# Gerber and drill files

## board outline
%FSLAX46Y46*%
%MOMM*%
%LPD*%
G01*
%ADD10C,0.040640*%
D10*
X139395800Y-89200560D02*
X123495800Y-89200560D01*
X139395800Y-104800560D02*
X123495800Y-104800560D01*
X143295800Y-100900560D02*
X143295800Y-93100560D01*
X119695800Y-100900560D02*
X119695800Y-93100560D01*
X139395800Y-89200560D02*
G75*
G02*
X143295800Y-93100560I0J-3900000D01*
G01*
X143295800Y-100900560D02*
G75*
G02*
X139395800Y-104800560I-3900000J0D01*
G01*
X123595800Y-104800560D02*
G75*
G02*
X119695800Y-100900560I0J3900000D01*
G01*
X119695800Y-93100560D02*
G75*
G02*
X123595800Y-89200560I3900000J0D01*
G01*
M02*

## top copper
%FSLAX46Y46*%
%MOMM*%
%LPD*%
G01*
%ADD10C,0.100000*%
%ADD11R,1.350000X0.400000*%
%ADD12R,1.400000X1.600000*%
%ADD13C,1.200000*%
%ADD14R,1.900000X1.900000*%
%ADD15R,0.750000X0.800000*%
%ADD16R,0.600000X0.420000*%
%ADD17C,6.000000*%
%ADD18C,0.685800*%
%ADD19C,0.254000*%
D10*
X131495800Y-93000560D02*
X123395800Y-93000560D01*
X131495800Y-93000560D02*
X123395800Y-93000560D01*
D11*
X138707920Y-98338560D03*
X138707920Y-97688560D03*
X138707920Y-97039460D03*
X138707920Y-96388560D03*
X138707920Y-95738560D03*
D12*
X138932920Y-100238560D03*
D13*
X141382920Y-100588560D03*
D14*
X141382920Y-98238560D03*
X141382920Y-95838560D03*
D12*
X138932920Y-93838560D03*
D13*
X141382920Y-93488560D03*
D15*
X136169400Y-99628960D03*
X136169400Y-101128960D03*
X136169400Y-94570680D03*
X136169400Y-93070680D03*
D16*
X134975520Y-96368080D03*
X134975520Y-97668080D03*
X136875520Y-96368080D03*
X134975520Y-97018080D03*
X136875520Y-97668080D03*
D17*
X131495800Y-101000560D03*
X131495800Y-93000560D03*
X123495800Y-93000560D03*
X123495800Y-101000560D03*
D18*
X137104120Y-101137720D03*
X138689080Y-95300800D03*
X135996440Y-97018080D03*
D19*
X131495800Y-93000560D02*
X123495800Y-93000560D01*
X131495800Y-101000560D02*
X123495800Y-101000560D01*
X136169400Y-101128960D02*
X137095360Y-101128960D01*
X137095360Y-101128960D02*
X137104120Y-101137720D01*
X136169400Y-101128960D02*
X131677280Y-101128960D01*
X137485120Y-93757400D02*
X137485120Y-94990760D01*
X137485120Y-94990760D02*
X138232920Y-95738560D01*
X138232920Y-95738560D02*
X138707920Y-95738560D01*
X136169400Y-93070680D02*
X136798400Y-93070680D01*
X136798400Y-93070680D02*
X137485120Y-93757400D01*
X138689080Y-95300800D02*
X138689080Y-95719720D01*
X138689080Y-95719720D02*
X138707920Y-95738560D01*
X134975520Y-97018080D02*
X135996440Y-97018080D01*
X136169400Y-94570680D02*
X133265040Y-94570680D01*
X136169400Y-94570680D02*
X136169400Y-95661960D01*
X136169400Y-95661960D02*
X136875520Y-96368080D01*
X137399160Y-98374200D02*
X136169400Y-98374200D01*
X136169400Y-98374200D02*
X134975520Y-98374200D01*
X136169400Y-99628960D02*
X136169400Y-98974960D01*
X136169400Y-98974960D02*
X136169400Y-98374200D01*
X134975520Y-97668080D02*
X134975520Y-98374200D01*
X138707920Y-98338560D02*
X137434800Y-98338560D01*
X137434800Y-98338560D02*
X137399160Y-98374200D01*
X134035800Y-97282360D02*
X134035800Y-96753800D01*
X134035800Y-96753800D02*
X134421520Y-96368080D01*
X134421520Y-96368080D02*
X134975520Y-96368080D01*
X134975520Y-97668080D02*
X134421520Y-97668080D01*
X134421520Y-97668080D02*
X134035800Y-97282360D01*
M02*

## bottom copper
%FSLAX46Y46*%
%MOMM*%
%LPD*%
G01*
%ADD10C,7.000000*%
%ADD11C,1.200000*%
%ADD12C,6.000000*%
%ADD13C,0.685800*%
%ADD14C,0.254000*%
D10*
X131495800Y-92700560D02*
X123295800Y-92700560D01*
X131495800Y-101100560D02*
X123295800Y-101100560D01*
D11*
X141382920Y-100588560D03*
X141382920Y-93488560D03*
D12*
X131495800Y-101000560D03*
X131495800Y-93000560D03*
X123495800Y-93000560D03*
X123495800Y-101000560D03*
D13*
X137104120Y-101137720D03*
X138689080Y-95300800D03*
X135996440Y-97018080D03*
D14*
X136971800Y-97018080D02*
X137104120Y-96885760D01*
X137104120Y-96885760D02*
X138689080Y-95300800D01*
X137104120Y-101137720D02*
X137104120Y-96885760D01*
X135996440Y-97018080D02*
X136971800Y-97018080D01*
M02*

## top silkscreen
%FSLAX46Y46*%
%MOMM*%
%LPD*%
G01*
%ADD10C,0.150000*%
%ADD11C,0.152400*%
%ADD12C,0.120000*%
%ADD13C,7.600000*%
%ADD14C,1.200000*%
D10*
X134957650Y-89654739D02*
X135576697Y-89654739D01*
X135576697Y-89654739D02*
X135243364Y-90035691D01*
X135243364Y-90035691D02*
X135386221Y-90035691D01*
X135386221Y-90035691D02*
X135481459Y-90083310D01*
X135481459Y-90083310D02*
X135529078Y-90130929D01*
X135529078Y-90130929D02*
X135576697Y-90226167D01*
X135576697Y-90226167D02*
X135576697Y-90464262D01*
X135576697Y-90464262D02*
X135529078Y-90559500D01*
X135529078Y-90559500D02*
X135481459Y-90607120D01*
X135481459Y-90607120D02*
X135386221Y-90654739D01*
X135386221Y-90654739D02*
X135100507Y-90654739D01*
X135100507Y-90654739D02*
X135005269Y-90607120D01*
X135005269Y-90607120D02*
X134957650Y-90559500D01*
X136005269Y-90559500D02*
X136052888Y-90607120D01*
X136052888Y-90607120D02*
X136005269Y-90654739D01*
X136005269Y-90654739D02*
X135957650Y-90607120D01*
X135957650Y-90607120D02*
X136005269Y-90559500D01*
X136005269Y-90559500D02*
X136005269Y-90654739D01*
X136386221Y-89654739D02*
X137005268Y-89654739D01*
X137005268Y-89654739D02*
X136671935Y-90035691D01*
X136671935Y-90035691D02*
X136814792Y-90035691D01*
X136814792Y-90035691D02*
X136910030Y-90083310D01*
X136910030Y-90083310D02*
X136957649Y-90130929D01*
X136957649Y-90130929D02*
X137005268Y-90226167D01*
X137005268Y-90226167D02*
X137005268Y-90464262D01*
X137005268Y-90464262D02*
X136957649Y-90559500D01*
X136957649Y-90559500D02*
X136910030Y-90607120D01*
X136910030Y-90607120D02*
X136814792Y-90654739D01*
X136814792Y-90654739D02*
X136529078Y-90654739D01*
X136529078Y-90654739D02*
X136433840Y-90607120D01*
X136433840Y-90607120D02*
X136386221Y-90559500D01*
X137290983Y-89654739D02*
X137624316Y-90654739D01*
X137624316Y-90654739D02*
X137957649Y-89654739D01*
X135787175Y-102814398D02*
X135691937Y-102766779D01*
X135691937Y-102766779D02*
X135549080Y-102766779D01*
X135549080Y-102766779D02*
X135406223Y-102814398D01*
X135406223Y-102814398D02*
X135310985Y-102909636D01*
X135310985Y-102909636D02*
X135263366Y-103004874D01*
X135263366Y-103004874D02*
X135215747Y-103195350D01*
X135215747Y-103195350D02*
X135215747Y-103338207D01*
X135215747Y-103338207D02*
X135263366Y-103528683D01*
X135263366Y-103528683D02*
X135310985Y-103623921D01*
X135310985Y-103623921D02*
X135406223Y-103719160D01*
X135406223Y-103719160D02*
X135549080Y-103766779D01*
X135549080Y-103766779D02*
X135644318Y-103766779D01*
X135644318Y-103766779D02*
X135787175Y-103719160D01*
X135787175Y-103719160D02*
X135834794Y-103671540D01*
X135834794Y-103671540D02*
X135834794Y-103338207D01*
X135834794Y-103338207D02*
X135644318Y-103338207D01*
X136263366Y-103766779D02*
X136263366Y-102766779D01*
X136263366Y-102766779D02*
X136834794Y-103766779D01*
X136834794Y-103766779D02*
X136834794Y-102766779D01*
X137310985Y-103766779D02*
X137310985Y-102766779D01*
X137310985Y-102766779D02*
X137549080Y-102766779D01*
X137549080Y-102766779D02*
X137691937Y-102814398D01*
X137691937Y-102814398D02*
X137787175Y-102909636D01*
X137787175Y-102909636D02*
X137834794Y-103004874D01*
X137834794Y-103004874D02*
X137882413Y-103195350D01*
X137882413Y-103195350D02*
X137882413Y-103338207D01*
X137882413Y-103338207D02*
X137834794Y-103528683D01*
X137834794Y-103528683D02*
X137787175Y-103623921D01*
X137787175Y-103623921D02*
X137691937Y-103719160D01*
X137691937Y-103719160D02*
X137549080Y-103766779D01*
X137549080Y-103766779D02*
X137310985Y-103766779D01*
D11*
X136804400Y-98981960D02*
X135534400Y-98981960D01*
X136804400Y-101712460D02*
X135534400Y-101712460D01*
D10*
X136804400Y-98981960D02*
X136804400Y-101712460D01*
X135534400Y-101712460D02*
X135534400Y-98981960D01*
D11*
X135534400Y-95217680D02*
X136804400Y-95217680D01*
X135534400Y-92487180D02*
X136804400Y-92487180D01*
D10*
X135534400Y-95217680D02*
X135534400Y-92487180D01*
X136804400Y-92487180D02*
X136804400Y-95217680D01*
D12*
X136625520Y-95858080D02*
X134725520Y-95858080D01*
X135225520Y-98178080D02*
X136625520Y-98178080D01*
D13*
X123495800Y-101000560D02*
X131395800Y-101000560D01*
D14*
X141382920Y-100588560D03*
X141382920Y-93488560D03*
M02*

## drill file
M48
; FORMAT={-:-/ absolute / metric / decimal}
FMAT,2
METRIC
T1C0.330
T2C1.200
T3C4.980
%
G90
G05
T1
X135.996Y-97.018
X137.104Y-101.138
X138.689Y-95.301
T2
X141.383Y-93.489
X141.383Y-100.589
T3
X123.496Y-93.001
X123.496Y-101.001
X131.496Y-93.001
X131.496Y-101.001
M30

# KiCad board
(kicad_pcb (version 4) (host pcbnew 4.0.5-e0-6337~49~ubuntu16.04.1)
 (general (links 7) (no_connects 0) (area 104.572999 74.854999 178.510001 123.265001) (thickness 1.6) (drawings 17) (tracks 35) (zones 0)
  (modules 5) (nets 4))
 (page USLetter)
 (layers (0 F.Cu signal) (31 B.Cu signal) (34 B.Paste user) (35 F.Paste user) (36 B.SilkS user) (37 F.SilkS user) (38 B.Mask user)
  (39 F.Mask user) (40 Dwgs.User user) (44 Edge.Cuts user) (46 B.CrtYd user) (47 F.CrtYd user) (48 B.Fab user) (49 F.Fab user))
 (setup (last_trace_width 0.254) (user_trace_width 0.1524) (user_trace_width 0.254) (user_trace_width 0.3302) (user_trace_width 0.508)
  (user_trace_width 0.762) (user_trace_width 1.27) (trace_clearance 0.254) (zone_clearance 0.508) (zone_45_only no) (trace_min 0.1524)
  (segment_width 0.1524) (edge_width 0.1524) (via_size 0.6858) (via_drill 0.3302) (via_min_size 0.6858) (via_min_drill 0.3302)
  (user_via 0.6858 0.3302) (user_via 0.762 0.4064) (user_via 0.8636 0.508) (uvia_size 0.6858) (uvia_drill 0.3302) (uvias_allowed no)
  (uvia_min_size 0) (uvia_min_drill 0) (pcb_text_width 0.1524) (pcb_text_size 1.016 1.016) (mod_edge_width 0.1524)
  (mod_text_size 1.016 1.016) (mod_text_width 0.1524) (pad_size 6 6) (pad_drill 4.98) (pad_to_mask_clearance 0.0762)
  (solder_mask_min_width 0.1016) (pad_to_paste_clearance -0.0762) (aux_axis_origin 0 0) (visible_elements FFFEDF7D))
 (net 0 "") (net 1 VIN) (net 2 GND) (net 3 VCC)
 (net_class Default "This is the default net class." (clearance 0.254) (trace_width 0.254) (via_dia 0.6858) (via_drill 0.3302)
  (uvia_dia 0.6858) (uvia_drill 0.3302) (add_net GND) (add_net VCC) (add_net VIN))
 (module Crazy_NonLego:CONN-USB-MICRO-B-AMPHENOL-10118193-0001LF (layer F.Cu) (at 141.38292 97.03856 90)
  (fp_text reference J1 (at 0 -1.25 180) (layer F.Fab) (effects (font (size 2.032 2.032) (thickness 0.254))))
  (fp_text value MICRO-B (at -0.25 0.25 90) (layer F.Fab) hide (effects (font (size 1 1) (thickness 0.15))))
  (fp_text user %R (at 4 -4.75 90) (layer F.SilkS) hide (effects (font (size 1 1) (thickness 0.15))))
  (pad 1 smd rect (at -1.3 -2.675 180) (size 1.35 0.4) (layers F.Cu F.Paste F.Mask) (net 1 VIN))
  (pad 2 smd rect (at -0.65 -2.675 180) (size 1.35 0.4) (layers F.Cu F.Paste F.Mask))
  (pad 3 smd rect (at -0.0009 -2.675 180) (size 1.35 0.4) (layers F.Cu F.Paste F.Mask))
  (pad 4 smd rect (at 0.65 -2.675 180) (size 1.35 0.4) (layers F.Cu F.Paste F.Mask))
  (pad 5 smd rect (at 1.3 -2.675 180) (size 1.35 0.4) (layers F.Cu F.Paste F.Mask) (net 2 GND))
  (pad 6 smd rect (at -3.2 -2.45 180) (size 1.4 1.6) (layers F.Cu F.Paste F.Mask))
  (pad 6 thru_hole circle (at -3.55 0 180) (size 1.2 1.2) (drill 1.2) (layers *.Cu *.Mask F.SilkS))
  (pad 6 smd rect (at -1.2 0 180) (size 1.9 1.9) (layers F.Cu F.Paste F.Mask))
  (pad 6 smd rect (at 1.2 0 180) (size 1.9 1.9) (layers F.Cu F.Paste F.Mask))
  (pad 6 smd rect (at 3.2 -2.45 180) (size 1.4 1.6) (layers F.Cu F.Paste F.Mask))
  (pad 6 thru_hole circle (at 3.55 0 180) (size 1.2 1.2) (drill 1.2) (layers *.Cu *.Mask F.SilkS)))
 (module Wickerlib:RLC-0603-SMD (layer F.Cu) (at 136.1694 100.37896 270)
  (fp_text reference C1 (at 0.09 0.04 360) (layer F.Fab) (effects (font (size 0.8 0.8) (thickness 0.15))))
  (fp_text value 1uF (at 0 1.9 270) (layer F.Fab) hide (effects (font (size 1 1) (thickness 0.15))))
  (fp_line (start -1.397 -0.635) (end -1.397 0.635) (layer F.SilkS) (width 0.1524))
  (fp_line (start 1.3335 -0.635) (end 1.3335 0.635) (layer F.SilkS) (width 0.1524))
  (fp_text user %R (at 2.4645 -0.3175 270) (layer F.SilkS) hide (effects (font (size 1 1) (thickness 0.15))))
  (fp_line (start -1.397 -0.635) (end 1.3335 -0.635) (layer F.SilkS) (width 0.15))
  (fp_line (start 1.3335 0.635) (end -1.397 0.635) (layer F.SilkS) (width 0.15))
  (pad 1 smd rect (at -0.75 0 270) (size 0.8 0.75) (layers F.Cu F.Paste F.Mask) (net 1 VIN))
  (pad 2 smd rect (at 0.75 0 270) (size 0.8 0.75) (layers F.Cu F.Paste F.Mask) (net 2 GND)))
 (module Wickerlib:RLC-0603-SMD (layer F.Cu) (at 136.1694 93.82068 90)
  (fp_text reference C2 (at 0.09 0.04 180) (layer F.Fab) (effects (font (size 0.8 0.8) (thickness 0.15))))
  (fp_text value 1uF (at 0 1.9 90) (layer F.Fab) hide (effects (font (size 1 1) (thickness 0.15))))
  (fp_line (start -1.397 -0.635) (end -1.397 0.635) (layer F.SilkS) (width 0.1524))
  (fp_line (start 1.3335 -0.635) (end 1.3335 0.635) (layer F.SilkS) (width 0.1524))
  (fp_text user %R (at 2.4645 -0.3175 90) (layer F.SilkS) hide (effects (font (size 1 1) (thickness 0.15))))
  (fp_line (start -1.397 -0.635) (end 1.3335 -0.635) (layer F.SilkS) (width 0.15))
  (fp_line (start 1.3335 0.635) (end -1.397 0.635) (layer F.SilkS) (width 0.15))
  (pad 1 smd rect (at -0.75 0 90) (size 0.8 0.75) (layers F.Cu F.Paste F.Mask) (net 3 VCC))
  (pad 2 smd rect (at 0.75 0 90) (size 0.8 0.75) (layers F.Cu F.Paste F.Mask) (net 2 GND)))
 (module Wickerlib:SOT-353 (layer F.Cu) (at 135.92552 97.01808)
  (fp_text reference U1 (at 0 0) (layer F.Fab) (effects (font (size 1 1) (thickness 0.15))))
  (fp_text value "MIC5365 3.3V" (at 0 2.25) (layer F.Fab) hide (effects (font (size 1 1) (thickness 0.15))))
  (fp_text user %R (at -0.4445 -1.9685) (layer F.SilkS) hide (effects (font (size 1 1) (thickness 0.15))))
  (fp_line (start 0.7 -1.16) (end -1.2 -1.16) (layer F.SilkS) (width 0.12))
  (fp_line (start -0.7 1.16) (end 0.7 1.16) (layer F.SilkS) (width 0.12))
  (pad 1 smd rect (at -0.95 -0.65) (size 0.6 0.42) (layers F.Cu F.Paste F.Mask) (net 1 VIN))
  (pad 3 smd rect (at -0.95 0.65) (size 0.6 0.42) (layers F.Cu F.Paste F.Mask) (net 1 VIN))
  (pad 5 smd rect (at 0.95 -0.65) (size 0.6 0.42) (layers F.Cu F.Paste F.Mask) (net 3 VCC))
  (pad 2 smd rect (at -0.95 0) (size 0.6 0.42) (layers F.Cu F.Paste F.Mask) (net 2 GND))
  (pad 4 smd rect (at 0.95 0.65) (size 0.6 0.42) (layers F.Cu F.Paste F.Mask)))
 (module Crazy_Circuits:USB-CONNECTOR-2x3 (layer F.Cu) (at 131.4958 101.00056)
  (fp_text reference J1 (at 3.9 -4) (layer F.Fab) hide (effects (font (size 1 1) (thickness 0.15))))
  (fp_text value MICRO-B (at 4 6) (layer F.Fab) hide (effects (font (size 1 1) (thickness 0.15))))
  (fp_line (start -8 0) (end -0.1 0) (layer F.SilkS) (width 7.6))
  (fp_line (start 0 -8.3) (end -8.2 -8.3) (layer B.Cu) (width 7))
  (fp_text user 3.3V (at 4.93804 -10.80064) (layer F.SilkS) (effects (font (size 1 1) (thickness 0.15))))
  (fp_line (start 7.9 -11.8) (end -8 -11.8) (layer Edge.Cuts) (width 0.04064))
  (fp_line (start 7.9 3.8) (end -8 3.8) (layer Edge.Cuts) (width 0.04064))
  (fp_line (start 11.8 -0.1) (end 11.8 -7.9) (layer Edge.Cuts) (width 0.04064))
  (fp_line (start -11.8 -0.1) (end -11.8 -7.9) (layer Edge.Cuts) (width 0.04064))
  (fp_arc (start 7.9 -7.9) (end 7.9 -11.8) (angle 90) (layer Edge.Cuts) (width 0.04064))
  (fp_arc (start 7.9 -0.1) (end 11.8 -0.1) (angle 90) (layer Edge.Cuts) (width 0.04064))
  (fp_arc (start -7.9 -0.1) (end -7.9 3.8) (angle 90) (layer Edge.Cuts) (width 0.04064))
  (fp_arc (start -7.9 -7.9) (end -11.8 -7.9) (angle 90) (layer Edge.Cuts) (width 0.04064))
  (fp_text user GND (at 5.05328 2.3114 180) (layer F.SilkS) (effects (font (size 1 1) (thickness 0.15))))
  (fp_line (start 0 0.1) (end -8.2 0.1) (layer B.Cu) (width 7))
  (fp_line (start 0 -8) (end -8.1 -8) (layer F.Cu) (width 0.1))
  (fp_line (start 0 -8) (end -8.1 -8) (layer F.Cu) (width 0.1))
  (pad 5 thru_hole circle (at 0 0) (size 6 6) (drill 4.98) (layers *.Cu *.Mask))
  (pad 1 thru_hole circle (at 0 -8) (size 6 6) (drill 4.98) (layers *.Cu *.Mask))
  (pad 1 thru_hole circle (at -8 -8) (size 6 6) (drill 4.98) (layers *.Cu *.Mask))
  (pad 5 thru_hole circle (at -8 0) (size 6 6) (drill 4.98) (layers *.Cu *.Mask)))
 (segment (start 131.4958 93.00056) (end 123.4958 93.00056) (width 0.254) (layer F.Cu) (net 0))
 (segment (start 131.4958 101.00056) (end 123.4958 101.00056) (width 0.254) (layer F.Cu) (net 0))
 (segment (start 136.9718 97.01808) (end 137.10412 96.88576) (width 0.254) (layer B.Cu) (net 2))
 (segment (start 137.10412 96.88576) (end 138.68908 95.3008) (width 0.254) (layer B.Cu) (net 2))
 (segment (start 137.10412 101.13772) (end 137.10412 96.88576) (width 0.254) (layer B.Cu) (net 2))
 (segment (start 136.1694 101.12896) (end 137.09536 101.12896) (width 0.254) (layer F.Cu) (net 2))
 (segment (start 137.09536 101.12896) (end 137.10412 101.13772) (width 0.254) (layer F.Cu) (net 2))
 (via (at 137.10412 101.13772) (size 0.6858) (drill 0.3302) (layers F.Cu B.Cu) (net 2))
 (segment (start 136.1694 101.12896) (end 131.67728 101.12896) (width 0.254) (layer F.Cu) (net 2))
 (segment (start 137.48512 93.7574) (end 137.48512 94.99076) (width 0.254) (layer F.Cu) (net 2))
 (segment (start 137.48512 94.99076) (end 138.23292 95.73856) (width 0.254) (layer F.Cu) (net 2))
 (segment (start 138.23292 95.73856) (end 138.70792 95.73856) (width 0.254) (layer F.Cu) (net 2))
 (segment (start 136.1694 93.07068) (end 136.7984 93.07068) (width 0.254) (layer F.Cu) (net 2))
 (segment (start 136.7984 93.07068) (end 137.48512 93.7574) (width 0.254) (layer F.Cu) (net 2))
 (segment (start 138.68908 95.3008) (end 138.68908 95.71972) (width 0.254) (layer F.Cu) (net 2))
 (segment (start 138.68908 95.71972) (end 138.70792 95.73856) (width 0.254) (layer F.Cu) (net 2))
 (via (at 138.68908 95.3008) (size 0.6858) (drill 0.3302) (layers F.Cu B.Cu) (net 2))
 (segment (start 135.99644 97.01808) (end 136.9718 97.01808) (width 0.254) (layer B.Cu) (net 2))
 (via (at 135.99644 97.01808) (size 0.6858) (drill 0.3302) (layers F.Cu B.Cu) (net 2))
 (segment (start 134.97552 97.01808) (end 135.99644 97.01808) (width 0.254) (layer F.Cu) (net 2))
 (segment (start 136.1694 94.57068) (end 133.26504 94.57068) (width 0.254) (layer F.Cu) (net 3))
 (segment (start 136.1694 94.57068) (end 136.1694 95.66196) (width 0.254) (layer F.Cu) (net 3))
 (segment (start 136.1694 95.66196) (end 136.87552 96.36808) (width 0.254) (layer F.Cu) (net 3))
 (segment (start 137.39916 98.3742) (end 136.1694 98.3742) (width 0.254) (layer F.Cu) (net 1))
 (segment (start 136.1694 98.3742) (end 134.97552 98.3742) (width 0.254) (layer F.Cu) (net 1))
 (segment (start 136.1694 99.62896) (end 136.1694 98.97496) (width 0.254) (layer F.Cu) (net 1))
 (segment (start 136.1694 98.97496) (end 136.1694 98.3742) (width 0.254) (layer F.Cu) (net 1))
 (segment (start 134.97552 97.66808) (end 134.97552 98.3742) (width 0.254) (layer F.Cu) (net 1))
 (segment (start 138.70792 98.33856) (end 137.4348 98.33856) (width 0.254) (layer F.Cu) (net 1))
 (segment (start 137.4348 98.33856) (end 137.39916 98.3742) (width 0.254) (layer F.Cu) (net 1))
 (segment (start 134.0358 97.28236) (end 134.0358 96.7538) (width 0.254) (layer F.Cu) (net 1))
 (segment (start 134.0358 96.7538) (end 134.42152 96.36808) (width 0.254) (layer F.Cu) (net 1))
 (segment (start 134.42152 96.36808) (end 134.97552 96.36808) (width 0.254) (layer F.Cu) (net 1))
 (segment (start 134.97552 97.66808) (end 134.42152 97.66808) (width 0.254) (layer F.Cu) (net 1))
 (segment (start 134.42152 97.66808) (end 134.0358 97.28236) (width 0.254) (layer F.Cu) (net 1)))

